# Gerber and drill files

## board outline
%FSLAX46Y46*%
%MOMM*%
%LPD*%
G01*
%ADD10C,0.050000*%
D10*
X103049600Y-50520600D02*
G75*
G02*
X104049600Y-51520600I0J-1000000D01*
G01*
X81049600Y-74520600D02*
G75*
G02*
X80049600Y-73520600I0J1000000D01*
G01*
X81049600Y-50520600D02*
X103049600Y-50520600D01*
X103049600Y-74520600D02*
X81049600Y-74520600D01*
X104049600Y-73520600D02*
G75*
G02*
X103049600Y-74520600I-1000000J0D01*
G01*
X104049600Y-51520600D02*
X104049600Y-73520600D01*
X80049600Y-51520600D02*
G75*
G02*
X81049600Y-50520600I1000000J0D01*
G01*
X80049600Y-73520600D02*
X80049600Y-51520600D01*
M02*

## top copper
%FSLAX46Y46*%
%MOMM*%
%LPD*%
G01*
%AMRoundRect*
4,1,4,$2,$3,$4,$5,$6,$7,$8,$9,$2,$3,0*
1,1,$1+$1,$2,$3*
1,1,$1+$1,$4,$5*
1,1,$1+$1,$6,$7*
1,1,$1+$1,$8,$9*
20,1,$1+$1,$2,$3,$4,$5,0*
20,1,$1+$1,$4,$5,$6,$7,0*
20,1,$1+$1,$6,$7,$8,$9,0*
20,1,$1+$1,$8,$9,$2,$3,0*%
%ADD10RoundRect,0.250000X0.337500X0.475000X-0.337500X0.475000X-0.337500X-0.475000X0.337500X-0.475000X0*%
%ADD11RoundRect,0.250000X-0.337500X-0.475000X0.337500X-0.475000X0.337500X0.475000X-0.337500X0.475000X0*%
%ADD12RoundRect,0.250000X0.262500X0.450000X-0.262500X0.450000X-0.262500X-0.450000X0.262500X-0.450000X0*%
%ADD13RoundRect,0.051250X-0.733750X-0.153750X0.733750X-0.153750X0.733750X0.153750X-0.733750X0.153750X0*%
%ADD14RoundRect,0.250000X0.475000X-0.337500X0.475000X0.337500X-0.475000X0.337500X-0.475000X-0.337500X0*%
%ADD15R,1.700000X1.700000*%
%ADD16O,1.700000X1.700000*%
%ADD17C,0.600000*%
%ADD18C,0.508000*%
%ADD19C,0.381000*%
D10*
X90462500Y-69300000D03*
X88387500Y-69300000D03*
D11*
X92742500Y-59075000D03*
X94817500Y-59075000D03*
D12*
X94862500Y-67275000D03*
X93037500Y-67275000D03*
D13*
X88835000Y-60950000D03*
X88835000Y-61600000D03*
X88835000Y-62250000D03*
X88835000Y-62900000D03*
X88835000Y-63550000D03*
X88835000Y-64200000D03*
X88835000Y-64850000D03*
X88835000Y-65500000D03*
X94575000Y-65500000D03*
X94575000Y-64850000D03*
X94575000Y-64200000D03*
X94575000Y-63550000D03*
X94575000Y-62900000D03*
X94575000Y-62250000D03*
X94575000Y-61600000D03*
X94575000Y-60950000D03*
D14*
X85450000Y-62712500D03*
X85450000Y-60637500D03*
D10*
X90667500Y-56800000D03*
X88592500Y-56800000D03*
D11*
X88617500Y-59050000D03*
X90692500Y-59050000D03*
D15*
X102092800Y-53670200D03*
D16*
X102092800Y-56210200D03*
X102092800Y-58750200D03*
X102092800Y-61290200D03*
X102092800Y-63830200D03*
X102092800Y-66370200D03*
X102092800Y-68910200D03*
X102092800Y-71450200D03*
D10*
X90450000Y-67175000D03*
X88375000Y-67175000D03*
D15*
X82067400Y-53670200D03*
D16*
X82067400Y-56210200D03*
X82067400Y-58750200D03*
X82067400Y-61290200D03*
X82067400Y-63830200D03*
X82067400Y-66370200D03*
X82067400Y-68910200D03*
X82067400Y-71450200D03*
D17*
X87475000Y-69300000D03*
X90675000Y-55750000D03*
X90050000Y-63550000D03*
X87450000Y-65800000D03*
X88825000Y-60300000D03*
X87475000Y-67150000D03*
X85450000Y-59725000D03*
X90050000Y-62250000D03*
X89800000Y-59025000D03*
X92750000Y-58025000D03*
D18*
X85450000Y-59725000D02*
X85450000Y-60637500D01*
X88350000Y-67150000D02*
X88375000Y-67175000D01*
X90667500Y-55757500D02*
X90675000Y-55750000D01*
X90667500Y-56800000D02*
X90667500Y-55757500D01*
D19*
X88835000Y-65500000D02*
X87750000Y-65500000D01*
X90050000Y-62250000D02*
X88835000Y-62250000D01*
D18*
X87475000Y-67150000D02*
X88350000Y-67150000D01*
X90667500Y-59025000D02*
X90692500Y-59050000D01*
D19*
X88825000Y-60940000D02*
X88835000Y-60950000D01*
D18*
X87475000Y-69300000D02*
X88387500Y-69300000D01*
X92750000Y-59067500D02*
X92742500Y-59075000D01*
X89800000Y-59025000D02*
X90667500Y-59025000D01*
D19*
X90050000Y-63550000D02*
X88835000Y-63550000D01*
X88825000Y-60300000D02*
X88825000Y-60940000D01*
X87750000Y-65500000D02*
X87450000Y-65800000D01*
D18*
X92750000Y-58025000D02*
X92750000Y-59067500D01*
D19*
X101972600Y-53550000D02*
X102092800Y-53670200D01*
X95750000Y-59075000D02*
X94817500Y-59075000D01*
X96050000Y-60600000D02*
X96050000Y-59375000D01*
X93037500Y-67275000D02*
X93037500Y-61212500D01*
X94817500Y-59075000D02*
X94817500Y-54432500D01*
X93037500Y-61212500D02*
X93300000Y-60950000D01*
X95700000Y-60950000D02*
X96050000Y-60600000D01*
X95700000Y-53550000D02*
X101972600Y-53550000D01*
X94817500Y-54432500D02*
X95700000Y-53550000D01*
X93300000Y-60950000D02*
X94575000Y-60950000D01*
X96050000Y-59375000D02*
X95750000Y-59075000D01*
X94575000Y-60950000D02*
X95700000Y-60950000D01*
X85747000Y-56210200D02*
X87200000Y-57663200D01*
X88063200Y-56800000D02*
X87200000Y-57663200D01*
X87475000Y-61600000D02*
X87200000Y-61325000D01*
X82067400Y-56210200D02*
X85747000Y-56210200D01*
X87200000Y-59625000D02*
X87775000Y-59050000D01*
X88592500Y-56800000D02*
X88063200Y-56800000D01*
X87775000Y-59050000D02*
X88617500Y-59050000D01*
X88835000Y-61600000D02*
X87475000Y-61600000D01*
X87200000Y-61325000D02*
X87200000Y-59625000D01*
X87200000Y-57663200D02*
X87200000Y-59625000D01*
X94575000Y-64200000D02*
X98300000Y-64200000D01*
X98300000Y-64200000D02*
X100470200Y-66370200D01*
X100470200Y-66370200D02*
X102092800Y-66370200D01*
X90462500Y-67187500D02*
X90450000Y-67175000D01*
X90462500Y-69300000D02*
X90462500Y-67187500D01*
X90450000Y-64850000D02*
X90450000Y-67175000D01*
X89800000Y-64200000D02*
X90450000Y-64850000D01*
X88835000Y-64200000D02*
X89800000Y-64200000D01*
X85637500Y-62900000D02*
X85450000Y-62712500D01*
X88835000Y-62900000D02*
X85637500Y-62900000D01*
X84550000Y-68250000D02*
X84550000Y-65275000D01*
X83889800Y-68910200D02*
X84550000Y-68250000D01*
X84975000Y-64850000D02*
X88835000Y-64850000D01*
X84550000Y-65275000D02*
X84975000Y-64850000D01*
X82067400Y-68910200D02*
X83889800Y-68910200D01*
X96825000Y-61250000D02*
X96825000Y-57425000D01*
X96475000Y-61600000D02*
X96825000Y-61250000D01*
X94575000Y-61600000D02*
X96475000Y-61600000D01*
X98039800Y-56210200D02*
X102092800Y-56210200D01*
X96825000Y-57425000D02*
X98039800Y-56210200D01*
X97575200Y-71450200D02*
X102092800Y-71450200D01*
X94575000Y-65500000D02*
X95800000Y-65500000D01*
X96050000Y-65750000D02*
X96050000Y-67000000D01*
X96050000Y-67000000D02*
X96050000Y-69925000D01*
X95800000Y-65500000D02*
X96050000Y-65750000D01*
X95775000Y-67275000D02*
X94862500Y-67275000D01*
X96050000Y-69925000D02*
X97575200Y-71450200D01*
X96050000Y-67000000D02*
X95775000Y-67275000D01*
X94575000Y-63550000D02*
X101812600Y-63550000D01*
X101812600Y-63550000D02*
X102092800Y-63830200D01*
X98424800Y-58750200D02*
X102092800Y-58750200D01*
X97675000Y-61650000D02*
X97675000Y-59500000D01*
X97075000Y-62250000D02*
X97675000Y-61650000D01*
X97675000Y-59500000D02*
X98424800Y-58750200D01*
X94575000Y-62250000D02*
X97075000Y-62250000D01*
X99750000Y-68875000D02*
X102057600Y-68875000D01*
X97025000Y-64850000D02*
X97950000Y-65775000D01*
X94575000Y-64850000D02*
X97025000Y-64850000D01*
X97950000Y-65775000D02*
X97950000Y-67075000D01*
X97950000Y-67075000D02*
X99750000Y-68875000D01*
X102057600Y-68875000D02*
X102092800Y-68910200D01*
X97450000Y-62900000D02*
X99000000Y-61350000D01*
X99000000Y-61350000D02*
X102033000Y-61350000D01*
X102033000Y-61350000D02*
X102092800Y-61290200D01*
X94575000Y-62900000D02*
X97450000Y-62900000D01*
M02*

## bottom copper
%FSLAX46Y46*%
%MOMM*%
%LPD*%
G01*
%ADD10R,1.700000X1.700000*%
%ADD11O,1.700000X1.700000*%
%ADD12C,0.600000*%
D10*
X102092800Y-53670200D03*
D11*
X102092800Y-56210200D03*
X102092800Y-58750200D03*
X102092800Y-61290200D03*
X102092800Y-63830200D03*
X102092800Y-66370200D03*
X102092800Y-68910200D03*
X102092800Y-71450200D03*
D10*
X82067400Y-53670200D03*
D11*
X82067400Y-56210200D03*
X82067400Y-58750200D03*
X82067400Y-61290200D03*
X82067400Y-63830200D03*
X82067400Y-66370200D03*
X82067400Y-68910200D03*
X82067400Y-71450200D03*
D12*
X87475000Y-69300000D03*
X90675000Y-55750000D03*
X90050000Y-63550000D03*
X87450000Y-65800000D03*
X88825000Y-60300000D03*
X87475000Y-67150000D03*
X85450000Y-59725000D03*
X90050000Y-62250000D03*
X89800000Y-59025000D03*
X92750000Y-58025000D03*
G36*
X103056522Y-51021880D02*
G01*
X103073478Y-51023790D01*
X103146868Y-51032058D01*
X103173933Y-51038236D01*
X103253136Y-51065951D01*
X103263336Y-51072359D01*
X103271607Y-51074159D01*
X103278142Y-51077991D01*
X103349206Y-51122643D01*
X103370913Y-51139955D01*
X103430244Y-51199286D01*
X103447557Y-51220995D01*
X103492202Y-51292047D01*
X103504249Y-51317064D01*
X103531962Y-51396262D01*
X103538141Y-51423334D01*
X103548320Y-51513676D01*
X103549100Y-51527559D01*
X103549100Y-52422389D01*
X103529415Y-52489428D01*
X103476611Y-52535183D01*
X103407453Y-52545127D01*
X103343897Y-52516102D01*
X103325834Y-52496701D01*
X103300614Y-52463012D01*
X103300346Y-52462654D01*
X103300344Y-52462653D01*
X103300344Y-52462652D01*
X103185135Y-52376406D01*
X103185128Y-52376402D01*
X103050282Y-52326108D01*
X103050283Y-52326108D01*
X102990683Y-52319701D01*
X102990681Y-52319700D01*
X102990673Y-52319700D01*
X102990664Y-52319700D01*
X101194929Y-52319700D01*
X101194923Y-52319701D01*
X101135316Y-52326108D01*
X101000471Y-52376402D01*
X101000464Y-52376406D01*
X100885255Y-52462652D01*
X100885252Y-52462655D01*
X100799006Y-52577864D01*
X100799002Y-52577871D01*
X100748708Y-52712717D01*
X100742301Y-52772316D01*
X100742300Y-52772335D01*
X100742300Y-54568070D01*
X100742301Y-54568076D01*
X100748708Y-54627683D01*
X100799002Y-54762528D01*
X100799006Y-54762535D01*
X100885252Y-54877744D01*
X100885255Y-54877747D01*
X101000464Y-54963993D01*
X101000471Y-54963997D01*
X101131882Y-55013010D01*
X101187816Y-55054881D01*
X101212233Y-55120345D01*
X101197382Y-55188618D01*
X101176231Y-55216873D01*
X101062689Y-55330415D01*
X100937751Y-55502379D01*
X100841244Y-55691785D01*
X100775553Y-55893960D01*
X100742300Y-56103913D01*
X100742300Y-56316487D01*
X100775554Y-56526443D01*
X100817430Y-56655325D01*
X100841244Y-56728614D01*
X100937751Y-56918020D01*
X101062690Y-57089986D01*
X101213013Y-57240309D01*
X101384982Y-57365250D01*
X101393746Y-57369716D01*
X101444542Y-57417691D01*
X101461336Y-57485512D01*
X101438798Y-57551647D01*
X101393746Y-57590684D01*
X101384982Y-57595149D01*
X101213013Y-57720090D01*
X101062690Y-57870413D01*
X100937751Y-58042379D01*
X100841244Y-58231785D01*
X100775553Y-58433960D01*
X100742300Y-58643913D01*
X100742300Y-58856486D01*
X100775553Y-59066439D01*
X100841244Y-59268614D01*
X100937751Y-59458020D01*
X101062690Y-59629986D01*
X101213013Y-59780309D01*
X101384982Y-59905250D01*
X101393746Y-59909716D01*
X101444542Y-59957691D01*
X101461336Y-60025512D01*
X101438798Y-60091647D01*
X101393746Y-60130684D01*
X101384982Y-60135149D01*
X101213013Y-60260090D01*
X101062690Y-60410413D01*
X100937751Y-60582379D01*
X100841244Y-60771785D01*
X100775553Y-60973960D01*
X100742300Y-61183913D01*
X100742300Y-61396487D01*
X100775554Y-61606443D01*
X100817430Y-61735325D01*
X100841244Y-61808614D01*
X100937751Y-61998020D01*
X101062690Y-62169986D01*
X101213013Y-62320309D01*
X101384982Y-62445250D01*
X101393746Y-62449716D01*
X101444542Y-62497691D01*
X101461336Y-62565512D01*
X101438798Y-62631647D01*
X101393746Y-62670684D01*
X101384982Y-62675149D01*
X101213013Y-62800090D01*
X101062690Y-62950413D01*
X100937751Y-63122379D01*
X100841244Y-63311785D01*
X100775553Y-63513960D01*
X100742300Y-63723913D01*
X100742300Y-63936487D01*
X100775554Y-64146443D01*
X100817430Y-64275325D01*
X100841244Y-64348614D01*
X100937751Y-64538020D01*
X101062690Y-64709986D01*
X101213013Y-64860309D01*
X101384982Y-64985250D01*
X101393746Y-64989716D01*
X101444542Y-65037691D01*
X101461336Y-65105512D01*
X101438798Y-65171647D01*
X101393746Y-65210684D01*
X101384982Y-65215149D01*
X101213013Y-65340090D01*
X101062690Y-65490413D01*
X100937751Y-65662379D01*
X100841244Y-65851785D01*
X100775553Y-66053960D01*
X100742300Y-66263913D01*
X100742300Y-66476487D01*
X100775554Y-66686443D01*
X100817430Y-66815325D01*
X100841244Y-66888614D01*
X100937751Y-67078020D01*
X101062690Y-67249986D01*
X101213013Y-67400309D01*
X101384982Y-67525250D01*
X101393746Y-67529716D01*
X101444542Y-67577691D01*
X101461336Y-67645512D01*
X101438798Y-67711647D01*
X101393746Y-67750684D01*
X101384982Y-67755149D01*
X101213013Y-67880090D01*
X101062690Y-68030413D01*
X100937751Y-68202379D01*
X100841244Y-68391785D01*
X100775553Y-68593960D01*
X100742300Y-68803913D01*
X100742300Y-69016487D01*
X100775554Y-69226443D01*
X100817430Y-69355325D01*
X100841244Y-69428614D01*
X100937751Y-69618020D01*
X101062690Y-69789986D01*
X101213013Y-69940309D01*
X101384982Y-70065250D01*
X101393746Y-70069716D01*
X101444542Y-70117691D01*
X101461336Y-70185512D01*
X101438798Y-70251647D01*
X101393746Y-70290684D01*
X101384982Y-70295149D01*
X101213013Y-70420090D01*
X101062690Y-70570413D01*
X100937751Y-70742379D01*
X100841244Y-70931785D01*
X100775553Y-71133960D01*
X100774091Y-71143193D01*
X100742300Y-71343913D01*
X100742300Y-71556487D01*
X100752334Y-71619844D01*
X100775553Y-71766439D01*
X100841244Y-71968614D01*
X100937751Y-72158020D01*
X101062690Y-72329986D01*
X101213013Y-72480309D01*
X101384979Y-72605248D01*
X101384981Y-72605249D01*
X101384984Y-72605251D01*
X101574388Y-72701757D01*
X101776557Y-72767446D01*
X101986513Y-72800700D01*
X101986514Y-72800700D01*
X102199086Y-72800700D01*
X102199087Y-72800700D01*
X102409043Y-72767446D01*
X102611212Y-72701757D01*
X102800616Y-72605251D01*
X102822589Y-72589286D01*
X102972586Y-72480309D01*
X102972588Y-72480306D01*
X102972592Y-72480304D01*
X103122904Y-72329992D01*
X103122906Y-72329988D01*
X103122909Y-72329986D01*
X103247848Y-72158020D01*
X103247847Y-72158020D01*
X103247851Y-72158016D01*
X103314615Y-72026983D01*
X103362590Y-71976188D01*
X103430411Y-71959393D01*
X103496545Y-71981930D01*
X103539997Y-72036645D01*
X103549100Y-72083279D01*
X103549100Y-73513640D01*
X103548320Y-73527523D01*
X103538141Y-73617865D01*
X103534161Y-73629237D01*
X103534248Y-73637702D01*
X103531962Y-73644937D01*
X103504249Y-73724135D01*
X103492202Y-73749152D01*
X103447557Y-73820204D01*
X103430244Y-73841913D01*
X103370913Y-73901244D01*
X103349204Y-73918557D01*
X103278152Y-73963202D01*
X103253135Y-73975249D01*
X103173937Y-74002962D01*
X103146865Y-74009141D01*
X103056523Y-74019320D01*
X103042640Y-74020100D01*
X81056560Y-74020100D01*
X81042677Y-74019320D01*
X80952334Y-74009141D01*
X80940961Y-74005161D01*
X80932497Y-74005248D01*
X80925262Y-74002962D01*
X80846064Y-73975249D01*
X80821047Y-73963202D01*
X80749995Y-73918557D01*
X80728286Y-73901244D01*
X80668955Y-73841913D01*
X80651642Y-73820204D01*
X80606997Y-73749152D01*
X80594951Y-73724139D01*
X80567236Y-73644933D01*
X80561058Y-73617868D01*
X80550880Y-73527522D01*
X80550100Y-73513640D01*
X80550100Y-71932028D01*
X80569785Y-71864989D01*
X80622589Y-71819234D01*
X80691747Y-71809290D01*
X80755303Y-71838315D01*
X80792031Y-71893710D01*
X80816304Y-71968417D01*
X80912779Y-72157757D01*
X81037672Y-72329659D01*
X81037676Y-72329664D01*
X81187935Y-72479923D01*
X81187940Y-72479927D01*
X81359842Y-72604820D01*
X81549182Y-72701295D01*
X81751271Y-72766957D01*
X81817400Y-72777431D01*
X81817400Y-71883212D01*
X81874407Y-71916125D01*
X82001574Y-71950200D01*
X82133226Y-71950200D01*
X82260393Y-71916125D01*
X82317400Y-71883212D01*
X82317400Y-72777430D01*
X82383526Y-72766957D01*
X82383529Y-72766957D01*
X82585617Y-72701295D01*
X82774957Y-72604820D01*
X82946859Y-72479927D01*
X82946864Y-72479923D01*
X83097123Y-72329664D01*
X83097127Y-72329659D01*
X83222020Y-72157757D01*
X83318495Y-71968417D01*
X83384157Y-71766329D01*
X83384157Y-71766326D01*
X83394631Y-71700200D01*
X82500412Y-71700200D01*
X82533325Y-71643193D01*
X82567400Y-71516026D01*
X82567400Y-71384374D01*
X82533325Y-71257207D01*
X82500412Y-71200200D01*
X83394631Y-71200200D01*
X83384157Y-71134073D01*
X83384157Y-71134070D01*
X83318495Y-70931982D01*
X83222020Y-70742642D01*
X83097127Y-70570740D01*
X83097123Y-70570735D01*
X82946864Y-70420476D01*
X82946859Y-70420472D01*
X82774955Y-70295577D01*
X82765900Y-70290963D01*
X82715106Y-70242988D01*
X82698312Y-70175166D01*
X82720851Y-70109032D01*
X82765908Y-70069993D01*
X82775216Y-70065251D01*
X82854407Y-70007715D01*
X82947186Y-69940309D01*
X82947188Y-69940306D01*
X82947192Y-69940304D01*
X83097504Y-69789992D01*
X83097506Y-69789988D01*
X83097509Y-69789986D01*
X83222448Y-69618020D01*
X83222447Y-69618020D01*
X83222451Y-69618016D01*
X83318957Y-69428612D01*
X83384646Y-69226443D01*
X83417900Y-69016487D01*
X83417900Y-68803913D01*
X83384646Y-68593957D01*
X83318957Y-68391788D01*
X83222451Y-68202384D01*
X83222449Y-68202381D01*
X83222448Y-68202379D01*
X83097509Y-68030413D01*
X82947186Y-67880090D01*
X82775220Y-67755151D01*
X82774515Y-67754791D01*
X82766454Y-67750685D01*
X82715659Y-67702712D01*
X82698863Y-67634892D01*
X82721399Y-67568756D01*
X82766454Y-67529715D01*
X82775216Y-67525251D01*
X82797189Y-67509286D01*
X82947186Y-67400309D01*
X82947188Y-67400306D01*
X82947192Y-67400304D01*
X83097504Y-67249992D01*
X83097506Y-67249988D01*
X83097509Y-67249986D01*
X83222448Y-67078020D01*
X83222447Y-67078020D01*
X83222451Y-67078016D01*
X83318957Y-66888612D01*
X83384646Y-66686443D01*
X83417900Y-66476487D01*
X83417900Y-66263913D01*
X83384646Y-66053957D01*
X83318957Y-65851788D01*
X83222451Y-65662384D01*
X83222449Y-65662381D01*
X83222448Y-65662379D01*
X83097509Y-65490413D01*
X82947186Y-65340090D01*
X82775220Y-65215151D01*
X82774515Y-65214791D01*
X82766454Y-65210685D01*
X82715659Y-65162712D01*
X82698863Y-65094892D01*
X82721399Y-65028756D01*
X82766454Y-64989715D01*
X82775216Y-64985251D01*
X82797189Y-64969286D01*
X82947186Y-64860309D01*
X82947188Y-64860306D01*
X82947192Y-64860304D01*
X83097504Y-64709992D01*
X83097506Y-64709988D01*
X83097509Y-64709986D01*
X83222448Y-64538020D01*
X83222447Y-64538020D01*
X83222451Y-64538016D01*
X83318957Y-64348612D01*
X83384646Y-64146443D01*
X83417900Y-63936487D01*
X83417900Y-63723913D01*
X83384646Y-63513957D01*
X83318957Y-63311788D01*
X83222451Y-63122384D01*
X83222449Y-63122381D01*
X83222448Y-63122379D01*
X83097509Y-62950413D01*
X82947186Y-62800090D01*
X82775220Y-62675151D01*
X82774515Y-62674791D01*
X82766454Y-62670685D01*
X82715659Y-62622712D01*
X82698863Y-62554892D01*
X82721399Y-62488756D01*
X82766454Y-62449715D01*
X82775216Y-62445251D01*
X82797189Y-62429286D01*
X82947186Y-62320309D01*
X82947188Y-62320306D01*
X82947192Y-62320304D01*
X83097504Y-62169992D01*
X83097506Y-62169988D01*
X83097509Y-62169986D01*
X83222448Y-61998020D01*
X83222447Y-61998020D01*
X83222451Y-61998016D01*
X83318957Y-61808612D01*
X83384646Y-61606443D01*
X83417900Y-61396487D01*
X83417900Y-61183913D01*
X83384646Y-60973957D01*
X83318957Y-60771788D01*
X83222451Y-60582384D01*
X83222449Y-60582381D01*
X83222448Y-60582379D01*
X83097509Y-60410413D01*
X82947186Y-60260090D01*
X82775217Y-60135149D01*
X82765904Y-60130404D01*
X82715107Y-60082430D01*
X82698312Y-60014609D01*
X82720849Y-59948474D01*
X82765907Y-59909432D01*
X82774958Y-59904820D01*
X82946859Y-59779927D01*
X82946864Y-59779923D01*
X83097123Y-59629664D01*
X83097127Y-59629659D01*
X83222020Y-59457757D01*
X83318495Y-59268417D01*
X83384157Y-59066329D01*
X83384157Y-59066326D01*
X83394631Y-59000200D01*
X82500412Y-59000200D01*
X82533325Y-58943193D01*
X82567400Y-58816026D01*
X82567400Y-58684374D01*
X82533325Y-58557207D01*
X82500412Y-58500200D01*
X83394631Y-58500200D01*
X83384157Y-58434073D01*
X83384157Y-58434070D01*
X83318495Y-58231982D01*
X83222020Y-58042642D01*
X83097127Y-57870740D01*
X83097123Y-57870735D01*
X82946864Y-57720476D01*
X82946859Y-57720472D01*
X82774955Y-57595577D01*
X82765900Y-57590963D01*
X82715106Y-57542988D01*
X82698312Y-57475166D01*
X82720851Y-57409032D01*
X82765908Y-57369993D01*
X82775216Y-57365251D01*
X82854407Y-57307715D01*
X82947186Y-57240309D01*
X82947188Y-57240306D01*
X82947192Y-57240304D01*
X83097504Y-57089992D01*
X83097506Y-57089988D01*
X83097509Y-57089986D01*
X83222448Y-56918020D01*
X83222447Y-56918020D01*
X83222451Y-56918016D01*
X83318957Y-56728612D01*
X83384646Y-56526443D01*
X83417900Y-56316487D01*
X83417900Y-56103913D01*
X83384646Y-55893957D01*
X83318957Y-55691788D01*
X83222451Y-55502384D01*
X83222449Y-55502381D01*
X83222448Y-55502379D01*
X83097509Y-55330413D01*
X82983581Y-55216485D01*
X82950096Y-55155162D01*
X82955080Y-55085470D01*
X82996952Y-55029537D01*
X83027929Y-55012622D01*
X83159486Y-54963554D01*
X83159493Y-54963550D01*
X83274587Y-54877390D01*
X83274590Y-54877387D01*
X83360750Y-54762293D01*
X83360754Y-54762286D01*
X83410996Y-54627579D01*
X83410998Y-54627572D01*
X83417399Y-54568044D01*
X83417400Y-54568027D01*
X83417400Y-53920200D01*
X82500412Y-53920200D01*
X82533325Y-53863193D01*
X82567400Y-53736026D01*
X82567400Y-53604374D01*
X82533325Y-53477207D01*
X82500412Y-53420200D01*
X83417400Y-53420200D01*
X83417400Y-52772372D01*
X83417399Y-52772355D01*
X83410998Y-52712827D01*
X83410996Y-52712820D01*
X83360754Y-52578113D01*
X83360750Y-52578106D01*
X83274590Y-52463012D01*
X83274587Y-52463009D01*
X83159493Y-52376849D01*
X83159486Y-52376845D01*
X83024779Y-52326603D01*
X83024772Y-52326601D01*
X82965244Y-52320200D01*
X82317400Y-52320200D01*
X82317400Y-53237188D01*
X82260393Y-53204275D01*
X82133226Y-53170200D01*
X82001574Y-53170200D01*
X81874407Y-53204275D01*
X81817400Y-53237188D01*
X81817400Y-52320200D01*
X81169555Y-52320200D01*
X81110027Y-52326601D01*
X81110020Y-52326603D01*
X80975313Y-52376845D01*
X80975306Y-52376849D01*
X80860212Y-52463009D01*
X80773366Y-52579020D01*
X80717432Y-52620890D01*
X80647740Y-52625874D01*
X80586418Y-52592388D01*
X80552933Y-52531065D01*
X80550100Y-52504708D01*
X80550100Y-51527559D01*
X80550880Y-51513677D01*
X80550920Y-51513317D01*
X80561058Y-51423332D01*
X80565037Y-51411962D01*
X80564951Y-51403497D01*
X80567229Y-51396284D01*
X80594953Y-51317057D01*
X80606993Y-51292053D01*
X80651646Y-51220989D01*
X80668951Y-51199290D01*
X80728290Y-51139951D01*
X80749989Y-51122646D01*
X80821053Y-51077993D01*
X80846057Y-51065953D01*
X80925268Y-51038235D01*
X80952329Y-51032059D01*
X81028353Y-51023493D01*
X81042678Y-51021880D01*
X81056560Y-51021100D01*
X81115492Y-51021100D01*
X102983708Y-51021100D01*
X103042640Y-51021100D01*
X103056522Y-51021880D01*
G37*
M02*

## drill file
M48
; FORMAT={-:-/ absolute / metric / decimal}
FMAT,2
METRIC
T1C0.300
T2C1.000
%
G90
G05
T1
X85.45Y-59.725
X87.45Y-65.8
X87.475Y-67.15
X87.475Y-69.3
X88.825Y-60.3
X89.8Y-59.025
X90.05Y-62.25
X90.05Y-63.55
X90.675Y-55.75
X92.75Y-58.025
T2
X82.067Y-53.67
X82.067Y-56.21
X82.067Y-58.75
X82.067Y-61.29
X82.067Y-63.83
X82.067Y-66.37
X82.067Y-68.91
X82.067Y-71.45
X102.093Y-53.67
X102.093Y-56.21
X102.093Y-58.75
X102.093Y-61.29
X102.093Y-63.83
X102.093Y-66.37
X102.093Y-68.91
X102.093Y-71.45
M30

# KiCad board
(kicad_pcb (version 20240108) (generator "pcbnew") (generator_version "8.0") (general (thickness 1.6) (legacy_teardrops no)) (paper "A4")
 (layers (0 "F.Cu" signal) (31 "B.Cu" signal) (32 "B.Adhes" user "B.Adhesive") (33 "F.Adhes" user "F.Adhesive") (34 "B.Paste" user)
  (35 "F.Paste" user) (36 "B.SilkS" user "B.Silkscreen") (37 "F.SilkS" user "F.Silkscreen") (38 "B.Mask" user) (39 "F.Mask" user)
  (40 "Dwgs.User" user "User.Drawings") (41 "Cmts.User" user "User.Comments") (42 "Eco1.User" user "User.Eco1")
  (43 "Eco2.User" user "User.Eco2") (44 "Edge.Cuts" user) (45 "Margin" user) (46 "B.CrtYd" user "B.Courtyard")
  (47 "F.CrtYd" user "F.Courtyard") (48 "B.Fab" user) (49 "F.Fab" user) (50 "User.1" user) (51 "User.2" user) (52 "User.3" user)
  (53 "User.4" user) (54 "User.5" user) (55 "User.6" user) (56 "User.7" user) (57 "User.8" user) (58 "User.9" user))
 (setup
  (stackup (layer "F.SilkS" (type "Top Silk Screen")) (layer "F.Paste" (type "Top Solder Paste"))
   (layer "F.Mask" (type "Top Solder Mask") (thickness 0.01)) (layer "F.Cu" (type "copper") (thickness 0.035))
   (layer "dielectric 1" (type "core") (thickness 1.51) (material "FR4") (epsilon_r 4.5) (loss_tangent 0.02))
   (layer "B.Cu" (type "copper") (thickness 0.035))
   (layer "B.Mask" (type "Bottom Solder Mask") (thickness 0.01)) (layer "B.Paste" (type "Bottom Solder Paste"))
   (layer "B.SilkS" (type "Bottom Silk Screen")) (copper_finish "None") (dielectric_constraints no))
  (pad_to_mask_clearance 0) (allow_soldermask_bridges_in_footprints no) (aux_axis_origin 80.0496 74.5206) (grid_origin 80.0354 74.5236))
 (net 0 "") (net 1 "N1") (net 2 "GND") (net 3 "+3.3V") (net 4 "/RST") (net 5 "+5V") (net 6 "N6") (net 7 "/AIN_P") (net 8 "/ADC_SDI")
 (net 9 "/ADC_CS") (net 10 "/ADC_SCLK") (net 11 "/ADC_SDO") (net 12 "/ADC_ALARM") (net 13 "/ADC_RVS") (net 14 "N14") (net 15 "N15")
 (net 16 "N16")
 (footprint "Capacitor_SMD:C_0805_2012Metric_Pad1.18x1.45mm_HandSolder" (layer "F.Cu") (at 89.425 69.3 180)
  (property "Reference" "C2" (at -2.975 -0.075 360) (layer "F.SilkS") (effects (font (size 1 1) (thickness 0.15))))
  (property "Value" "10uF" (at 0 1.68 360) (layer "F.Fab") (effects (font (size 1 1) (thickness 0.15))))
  (pad "1" smd roundrect (at -1.0375 0 180) (size 1.175 1.45) (layers "F.Cu" "F.Paste" "F.Mask") (roundrect_rratio 0.212766) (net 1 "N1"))
  (pad "2" smd roundrect (at 1.0375 0 180) (size 1.175 1.45) (layers "F.Cu" "F.Paste" "F.Mask") (roundrect_rratio 0.212766) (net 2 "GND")))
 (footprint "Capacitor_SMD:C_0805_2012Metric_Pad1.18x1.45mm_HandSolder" (layer "F.Cu") (at 93.78 59.075)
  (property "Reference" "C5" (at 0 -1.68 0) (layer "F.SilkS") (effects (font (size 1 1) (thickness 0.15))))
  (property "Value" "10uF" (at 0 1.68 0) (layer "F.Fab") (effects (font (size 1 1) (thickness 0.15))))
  (pad "1" smd roundrect (at -1.0375 0) (size 1.175 1.45) (layers "F.Cu" "F.Paste" "F.Mask") (roundrect_rratio 0.212766) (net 2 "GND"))
  (pad "2" smd roundrect (at 1.0375 0) (size 1.175 1.45) (layers "F.Cu" "F.Paste" "F.Mask") (roundrect_rratio 0.212766) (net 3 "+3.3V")))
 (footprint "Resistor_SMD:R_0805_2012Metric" (layer "F.Cu") (at 93.95 67.275 180)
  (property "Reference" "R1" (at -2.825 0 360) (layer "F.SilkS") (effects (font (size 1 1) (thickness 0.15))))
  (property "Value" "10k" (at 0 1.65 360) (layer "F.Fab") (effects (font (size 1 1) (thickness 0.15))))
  (pad "1" smd roundrect (at -0.9125 0 180) (size 1.025 1.4) (layers "F.Cu" "F.Paste" "F.Mask") (roundrect_rratio 0.243902) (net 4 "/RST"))
  (pad "2" smd roundrect (at 0.9125 0 180) (size 1.025 1.4) (layers "F.Cu" "F.Paste" "F.Mask") (roundrect_rratio 0.243902) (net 3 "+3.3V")))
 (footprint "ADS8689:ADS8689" (layer "F.Cu") (at 91.705 63.225)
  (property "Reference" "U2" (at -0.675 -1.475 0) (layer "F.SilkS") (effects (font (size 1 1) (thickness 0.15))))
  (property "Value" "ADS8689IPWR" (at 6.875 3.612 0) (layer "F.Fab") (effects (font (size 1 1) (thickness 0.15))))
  (pad "1" smd roundrect (at -2.87 -2.275) (size 1.57 0.41) (layers "F.Cu" "F.Paste" "F.Mask") (roundrect_rratio 0.125) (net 2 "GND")
   (solder_mask_margin 0.102))
  (pad "2" smd roundrect (at -2.87 -1.625) (size 1.57 0.41) (layers "F.Cu" "F.Paste" "F.Mask") (roundrect_rratio 0.125) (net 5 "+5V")
   (solder_mask_margin 0.102))
  (pad "3" smd roundrect (at -2.87 -0.975) (size 1.57 0.41) (layers "F.Cu" "F.Paste" "F.Mask") (roundrect_rratio 0.125) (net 2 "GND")
   (solder_mask_margin 0.102))
  (pad "4" smd roundrect (at -2.87 -0.325) (size 1.57 0.41) (layers "F.Cu" "F.Paste" "F.Mask") (roundrect_rratio 0.125) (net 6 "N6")
   (solder_mask_margin 0.102))
  (pad "5" smd roundrect (at -2.87 0.325) (size 1.57 0.41) (layers "F.Cu" "F.Paste" "F.Mask") (roundrect_rratio 0.125) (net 2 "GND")
   (solder_mask_margin 0.102))
  (pad "6" smd roundrect (at -2.87 0.975) (size 1.57 0.41) (layers "F.Cu" "F.Paste" "F.Mask") (roundrect_rratio 0.125) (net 1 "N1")
   (solder_mask_margin 0.102))
  (pad "7" smd roundrect (at -2.87 1.625) (size 1.57 0.41) (layers "F.Cu" "F.Paste" "F.Mask") (roundrect_rratio 0.125) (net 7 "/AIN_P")
   (solder_mask_margin 0.102))
  (pad "8" smd roundrect (at -2.87 2.275) (size 1.57 0.41) (layers "F.Cu" "F.Paste" "F.Mask") (roundrect_rratio 0.125) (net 2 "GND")
   (solder_mask_margin 0.102))
  (pad "9" smd roundrect (at 2.87 2.275) (size 1.57 0.41) (layers "F.Cu" "F.Paste" "F.Mask") (roundrect_rratio 0.125) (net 4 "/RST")
   (solder_mask_margin 0.102))
  (pad "10" smd roundrect (at 2.87 1.625) (size 1.57 0.41) (layers "F.Cu" "F.Paste" "F.Mask") (roundrect_rratio 0.125) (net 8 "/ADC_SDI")
   (solder_mask_margin 0.102))
  (pad "11" smd roundrect (at 2.87 0.975) (size 1.57 0.41) (layers "F.Cu" "F.Paste" "F.Mask") (roundrect_rratio 0.125) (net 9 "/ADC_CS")
   (solder_mask_margin 0.102))
  (pad "12" smd roundrect (at 2.87 0.325) (size 1.57 0.41) (layers "F.Cu" "F.Paste" "F.Mask") (roundrect_rratio 0.125) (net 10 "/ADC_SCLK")
   (solder_mask_margin 0.102))
  (pad "13" smd roundrect (at 2.87 -0.325) (size 1.57 0.41) (layers "F.Cu" "F.Paste" "F.Mask") (roundrect_rratio 0.125) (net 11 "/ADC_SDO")
   (solder_mask_margin 0.102))
  (pad "14" smd roundrect (at 2.87 -0.975) (size 1.57 0.41) (layers "F.Cu" "F.Paste" "F.Mask") (roundrect_rratio 0.125)
   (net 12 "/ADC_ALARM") (solder_mask_margin 0.102))
  (pad "15" smd roundrect (at 2.87 -1.625) (size 1.57 0.41) (layers "F.Cu" "F.Paste" "F.Mask") (roundrect_rratio 0.125) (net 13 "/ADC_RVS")
   (solder_mask_margin 0.102))
  (pad "16" smd roundrect (at 2.87 -2.275) (size 1.57 0.41) (layers "F.Cu" "F.Paste" "F.Mask") (roundrect_rratio 0.125) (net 3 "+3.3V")
   (solder_mask_margin 0.102)))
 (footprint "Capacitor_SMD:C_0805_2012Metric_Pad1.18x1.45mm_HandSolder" (layer "F.Cu") (at 85.45 61.675 90)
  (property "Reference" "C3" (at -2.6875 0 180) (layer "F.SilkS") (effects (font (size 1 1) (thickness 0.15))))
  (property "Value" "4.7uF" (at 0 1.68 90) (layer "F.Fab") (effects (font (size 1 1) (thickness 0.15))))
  (pad "1" smd roundrect (at -1.0375 0 90) (size 1.175 1.45) (layers "F.Cu" "F.Paste" "F.Mask") (roundrect_rratio 0.212766) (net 6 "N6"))
  (pad "2" smd roundrect (at 1.0375 0 90) (size 1.175 1.45) (layers "F.Cu" "F.Paste" "F.Mask") (roundrect_rratio 0.212766) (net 2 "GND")))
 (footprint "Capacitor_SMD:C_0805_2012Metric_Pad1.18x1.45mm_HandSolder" (layer "F.Cu") (at 89.63 56.8 180)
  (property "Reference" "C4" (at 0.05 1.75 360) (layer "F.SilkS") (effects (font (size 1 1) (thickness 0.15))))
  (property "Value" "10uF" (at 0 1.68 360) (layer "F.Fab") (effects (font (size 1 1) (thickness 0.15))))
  (pad "1" smd roundrect (at -1.0375 0 180) (size 1.175 1.45) (layers "F.Cu" "F.Paste" "F.Mask") (roundrect_rratio 0.212766) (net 2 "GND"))
  (pad "2" smd roundrect (at 1.0375 0 180) (size 1.175 1.45) (layers "F.Cu" "F.Paste" "F.Mask") (roundrect_rratio 0.212766) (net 5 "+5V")))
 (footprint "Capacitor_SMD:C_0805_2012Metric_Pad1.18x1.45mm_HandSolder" (layer "F.Cu") (at 89.655 59.05)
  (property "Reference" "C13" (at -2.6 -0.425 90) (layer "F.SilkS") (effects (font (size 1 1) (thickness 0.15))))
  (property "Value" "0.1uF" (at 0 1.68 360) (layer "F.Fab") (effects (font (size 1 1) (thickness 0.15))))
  (pad "1" smd roundrect (at -1.0375 0) (size 1.175 1.45) (layers "F.Cu" "F.Paste" "F.Mask") (roundrect_rratio 0.212766) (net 5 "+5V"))
  (pad "2" smd roundrect (at 1.0375 0) (size 1.175 1.45) (layers "F.Cu" "F.Paste" "F.Mask") (roundrect_rratio 0.212766) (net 2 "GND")))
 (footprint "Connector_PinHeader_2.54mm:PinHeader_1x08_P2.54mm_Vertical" (layer "F.Cu") (at 102.0928 53.6702)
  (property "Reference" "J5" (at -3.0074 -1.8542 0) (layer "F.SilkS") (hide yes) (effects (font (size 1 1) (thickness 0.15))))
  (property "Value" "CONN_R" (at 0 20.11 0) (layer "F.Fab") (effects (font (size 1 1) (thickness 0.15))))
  (pad "1" thru_hole rect (at 0 0) (size 1.7 1.7) (drill 1) (layers "*.Cu" "*.Mask") (remove_unused_layers no) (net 3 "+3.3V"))
  (pad "2" thru_hole oval (at 0 2.54) (size 1.7 1.7) (drill 1) (layers "*.Cu" "*.Mask") (remove_unused_layers no) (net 13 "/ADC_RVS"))
  (pad "3" thru_hole oval (at 0 5.08) (size 1.7 1.7) (drill 1) (layers "*.Cu" "*.Mask") (remove_unused_layers no) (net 12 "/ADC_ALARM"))
  (pad "4" thru_hole oval (at 0 7.62) (size 1.7 1.7) (drill 1) (layers "*.Cu" "*.Mask") (remove_unused_layers no) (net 11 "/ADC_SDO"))
  (pad "5" thru_hole oval (at 0 10.16) (size 1.7 1.7) (drill 1) (layers "*.Cu" "*.Mask") (remove_unused_layers no) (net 10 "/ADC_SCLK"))
  (pad "6" thru_hole oval (at 0 12.7) (size 1.7 1.7) (drill 1) (layers "*.Cu" "*.Mask") (remove_unused_layers no) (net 9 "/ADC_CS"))
  (pad "7" thru_hole oval (at 0 15.24) (size 1.7 1.7) (drill 1) (layers "*.Cu" "*.Mask") (remove_unused_layers no) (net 8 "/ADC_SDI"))
  (pad "8" thru_hole oval (at 0 17.78) (size 1.7 1.7) (drill 1) (layers "*.Cu" "*.Mask") (remove_unused_layers no) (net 4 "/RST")))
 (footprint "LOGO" (layer "F.Cu") (at 96.125 54.1)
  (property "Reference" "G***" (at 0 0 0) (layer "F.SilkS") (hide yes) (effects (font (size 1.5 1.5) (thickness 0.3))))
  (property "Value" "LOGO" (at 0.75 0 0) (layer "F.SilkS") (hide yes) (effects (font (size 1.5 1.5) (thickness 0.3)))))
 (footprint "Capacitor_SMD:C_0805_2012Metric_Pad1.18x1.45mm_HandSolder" (layer "F.Cu") (at 89.4125 67.175 180)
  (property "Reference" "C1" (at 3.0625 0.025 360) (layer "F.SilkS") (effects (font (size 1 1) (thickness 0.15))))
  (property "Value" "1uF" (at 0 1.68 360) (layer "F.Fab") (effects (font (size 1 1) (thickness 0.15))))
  (pad "1" smd roundrect (at -1.0375 0 180) (size 1.175 1.45) (layers "F.Cu" "F.Paste" "F.Mask") (roundrect_rratio 0.212766) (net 1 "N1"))
  (pad "2" smd roundrect (at 1.0375 0 180) (size 1.175 1.45) (layers "F.Cu" "F.Paste" "F.Mask") (roundrect_rratio 0.212766) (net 2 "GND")))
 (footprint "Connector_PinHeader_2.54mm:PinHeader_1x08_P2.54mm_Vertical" (layer "F.Cu") (at 82.0674 53.6702)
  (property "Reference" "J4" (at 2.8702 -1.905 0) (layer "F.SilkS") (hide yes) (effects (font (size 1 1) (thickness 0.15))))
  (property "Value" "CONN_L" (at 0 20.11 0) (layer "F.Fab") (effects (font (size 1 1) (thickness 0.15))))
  (pad "1" thru_hole rect (at 0 0) (size 1.7 1.7) (drill 1) (layers "*.Cu" "*.Mask") (remove_unused_layers no) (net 2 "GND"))
  (pad "2" thru_hole oval (at 0 2.54) (size 1.7 1.7) (drill 1) (layers "*.Cu" "*.Mask") (remove_unused_layers no) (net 5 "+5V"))
  (pad "3" thru_hole oval (at 0 5.08) (size 1.7 1.7) (drill 1) (layers "*.Cu" "*.Mask") (remove_unused_layers no) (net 2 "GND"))
  (pad "4" thru_hole oval (at 0 7.62) (size 1.7 1.7) (drill 1) (layers "*.Cu" "*.Mask") (remove_unused_layers no) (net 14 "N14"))
  (pad "5" thru_hole oval (at 0 10.16) (size 1.7 1.7) (drill 1) (layers "*.Cu" "*.Mask") (remove_unused_layers no) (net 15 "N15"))
  (pad "6" thru_hole oval (at 0 12.7) (size 1.7 1.7) (drill 1) (layers "*.Cu" "*.Mask") (remove_unused_layers no) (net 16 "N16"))
  (pad "7" thru_hole oval (at 0 15.24) (size 1.7 1.7) (drill 1) (layers "*.Cu" "*.Mask") (remove_unused_layers no) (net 7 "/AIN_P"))
  (pad "8" thru_hole oval (at 0 17.78) (size 1.7 1.7) (drill 1) (layers "*.Cu" "*.Mask") (remove_unused_layers no) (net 2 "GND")))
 (gr_arc (start 103.0496 50.5206) (mid 103.756707 50.813493) (end 104.0496 51.5206) (stroke (width 0.05) (type default)) (layer "Edge.Cuts"))
 (gr_arc (start 81.0496 74.5206) (mid 80.342493 74.227707) (end 80.0496 73.5206) (stroke (width 0.05) (type default)) (layer "Edge.Cuts"))
 (gr_line (start 81.0496 50.5206) (end 103.0496 50.5206) (stroke (width 0.05) (type default)) (layer "Edge.Cuts"))
 (gr_line (start 103.0496 74.5206) (end 81.0496 74.5206) (stroke (width 0.05) (type default)) (layer "Edge.Cuts"))
 (gr_arc (start 104.0496 73.5206) (mid 103.756707 74.227707) (end 103.0496 74.5206) (stroke (width 0.05) (type default)) (layer "Edge.Cuts"))
 (gr_line (start 104.0496 51.5206) (end 104.0496 73.5206) (stroke (width 0.05) (type default)) (layer "Edge.Cuts"))
 (gr_arc (start 80.0496 51.5206) (mid 80.342493 50.813493) (end 81.0496 50.5206) (stroke (width 0.05) (type default)) (layer "Edge.Cuts"))
 (gr_line (start 80.0496 73.5206) (end 80.0496 51.5206) (stroke (width 0.05) (type default)) (layer "Edge.Cuts"))
 (segment (start 85.45 59.725) (end 85.45 60.6375) (width 0.508) (layer "F.Cu") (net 2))
 (segment (start 88.35 67.15) (end 88.375 67.175) (width 0.508) (layer "F.Cu") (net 2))
 (segment (start 90.6675 55.7575) (end 90.675 55.75) (width 0.508) (layer "F.Cu") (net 2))
 (segment (start 90.6675 56.8) (end 90.6675 55.7575) (width 0.508) (layer "F.Cu") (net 2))
 (segment (start 88.835 65.5) (end 87.75 65.5) (width 0.381) (layer "F.Cu") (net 2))
 (segment (start 90.05 62.25) (end 88.835 62.25) (width 0.381) (layer "F.Cu") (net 2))
 (segment (start 87.475 67.15) (end 88.35 67.15) (width 0.508) (layer "F.Cu") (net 2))
 (segment (start 90.6675 59.025) (end 90.6925 59.05) (width 0.508) (layer "F.Cu") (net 2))
 (segment (start 88.825 60.94) (end 88.835 60.95) (width 0.381) (layer "F.Cu") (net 2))
 (segment (start 87.475 69.3) (end 88.3875 69.3) (width 0.508) (layer "F.Cu") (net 2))
 (segment (start 92.75 59.0675) (end 92.7425 59.075) (width 0.508) (layer "F.Cu") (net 2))
 (segment (start 89.8 59.025) (end 90.6675 59.025) (width 0.508) (layer "F.Cu") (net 2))
 (segment (start 90.05 63.55) (end 88.835 63.55) (width 0.381) (layer "F.Cu") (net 2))
 (segment (start 88.825 60.3) (end 88.825 60.94) (width 0.381) (layer "F.Cu") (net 2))
 (segment (start 87.75 65.5) (end 87.45 65.8) (width 0.381) (layer "F.Cu") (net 2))
 (segment (start 92.75 58.025) (end 92.75 59.0675) (width 0.508) (layer "F.Cu") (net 2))
 (via (at 87.475 69.3) (size 0.6) (drill 0.3) (layers "F.Cu" "B.Cu") (free yes) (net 2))
 (via (at 90.675 55.75) (size 0.6) (drill 0.3) (layers "F.Cu" "B.Cu") (free yes) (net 2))
 (via (at 90.05 63.55) (size 0.6) (drill 0.3) (layers "F.Cu" "B.Cu") (free yes) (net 2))
 (via (at 87.45 65.8) (size 0.6) (drill 0.3) (layers "F.Cu" "B.Cu") (free yes) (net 2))
 (via (at 88.825 60.3) (size 0.6) (drill 0.3) (layers "F.Cu" "B.Cu") (free yes) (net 2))
 (via (at 87.475 67.15) (size 0.6) (drill 0.3) (layers "F.Cu" "B.Cu") (free yes) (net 2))
 (via (at 85.45 59.725) (size 0.6) (drill 0.3) (layers "F.Cu" "B.Cu") (free yes) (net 2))
 (via (at 90.05 62.25) (size 0.6) (drill 0.3) (layers "F.Cu" "B.Cu") (free yes) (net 2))
 (via (at 89.8 59.025) (size 0.6) (drill 0.3) (layers "F.Cu" "B.Cu") (free yes) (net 2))
 (via (at 92.75 58.025) (size 0.6) (drill 0.3) (layers "F.Cu" "B.Cu") (free yes) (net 2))
 (segment (start 101.9726 53.55) (end 102.0928 53.6702) (width 0.381) (layer "F.Cu") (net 3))
 (segment (start 95.75 59.075) (end 94.8175 59.075) (width 0.381) (layer "F.Cu") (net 3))
 (segment (start 96.05 60.6) (end 96.05 59.375) (width 0.381) (layer "F.Cu") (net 3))
 (segment (start 93.0375 67.275) (end 93.0375 61.2125) (width 0.381) (layer "F.Cu") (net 3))
 (segment (start 94.8175 59.075) (end 94.8175 54.4325) (width 0.381) (layer "F.Cu") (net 3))
 (segment (start 93.0375 61.2125) (end 93.3 60.95) (width 0.381) (layer "F.Cu") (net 3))
 (segment (start 95.7 60.95) (end 96.05 60.6) (width 0.381) (layer "F.Cu") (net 3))
 (segment (start 95.7 53.55) (end 101.9726 53.55) (width 0.381) (layer "F.Cu") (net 3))
 (segment (start 94.8175 54.4325) (end 95.7 53.55) (width 0.381) (layer "F.Cu") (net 3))
 (segment (start 93.3 60.95) (end 94.575 60.95) (width 0.381) (layer "F.Cu") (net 3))
 (segment (start 96.05 59.375) (end 95.75 59.075) (width 0.381) (layer "F.Cu") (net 3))
 (segment (start 94.575 60.95) (end 95.7 60.95) (width 0.381) (layer "F.Cu") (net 3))
 (segment (start 85.747 56.2102) (end 87.2 57.6632) (width 0.381) (layer "F.Cu") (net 5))
 (segment (start 88.0632 56.8) (end 87.2 57.6632) (width 0.381) (layer "F.Cu") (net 5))
 (segment (start 87.475 61.6) (end 87.2 61.325) (width 0.381) (layer "F.Cu") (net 5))
 (segment (start 82.0674 56.2102) (end 85.747 56.2102) (width 0.381) (layer "F.Cu") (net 5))
 (segment (start 87.2 59.625) (end 87.775 59.05) (width 0.381) (layer "F.Cu") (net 5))
 (segment (start 88.5925 56.8) (end 88.0632 56.8) (width 0.381) (layer "F.Cu") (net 5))
 (segment (start 87.775 59.05) (end 88.6175 59.05) (width 0.381) (layer "F.Cu") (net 5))
 (segment (start 88.835 61.6) (end 87.475 61.6) (width 0.381) (layer "F.Cu") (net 5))
 (segment (start 87.2 61.325) (end 87.2 59.625) (width 0.381) (layer "F.Cu") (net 5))
 (segment (start 87.2 57.6632) (end 87.2 59.625) (width 0.381) (layer "F.Cu") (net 5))
 (segment (start 94.575 64.2) (end 98.3 64.2) (width 0.381) (layer "F.Cu") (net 9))
 (segment (start 98.3 64.2) (end 100.4702 66.3702) (width 0.381) (layer "F.Cu") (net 9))
 (segment (start 100.4702 66.3702) (end 102.0928 66.3702) (width 0.381) (layer "F.Cu") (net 9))
 (segment (start 90.4625 67.1875) (end 90.45 67.175) (width 0.381) (layer "F.Cu") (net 1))
 (segment (start 90.4625 69.3) (end 90.4625 67.1875) (width 0.381) (layer "F.Cu") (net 1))
 (segment (start 90.45 64.85) (end 90.45 67.175) (width 0.381) (layer "F.Cu") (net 1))
 (segment (start 89.8 64.2) (end 90.45 64.85) (width 0.381) (layer "F.Cu") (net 1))
 (segment (start 88.835 64.2) (end 89.8 64.2) (width 0.381) (layer "F.Cu") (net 1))
 (segment (start 85.6375 62.9) (end 85.45 62.7125) (width 0.381) (layer "F.Cu") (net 6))
 (segment (start 88.835 62.9) (end 85.6375 62.9) (width 0.381) (layer "F.Cu") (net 6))
 (segment (start 84.55 68.25) (end 84.55 65.275) (width 0.381) (layer "F.Cu") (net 7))
 (segment (start 83.8898 68.9102) (end 84.55 68.25) (width 0.381) (layer "F.Cu") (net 7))
 (segment (start 84.975 64.85) (end 88.835 64.85) (width 0.381) (layer "F.Cu") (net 7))
 (segment (start 84.55 65.275) (end 84.975 64.85) (width 0.381) (layer "F.Cu") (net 7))
 (segment (start 82.0674 68.9102) (end 83.8898 68.9102) (width 0.381) (layer "F.Cu") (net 7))
 (segment (start 96.825 61.25) (end 96.825 57.425) (width 0.381) (layer "F.Cu") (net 13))
 (segment (start 96.475 61.6) (end 96.825 61.25) (width 0.381) (layer "F.Cu") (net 13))
 (segment (start 94.575 61.6) (end 96.475 61.6) (width 0.381) (layer "F.Cu") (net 13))
 (segment (start 98.0398 56.2102) (end 102.0928 56.2102) (width 0.381) (layer "F.Cu") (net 13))
 (segment (start 96.825 57.425) (end 98.0398 56.2102) (width 0.381) (layer "F.Cu") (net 13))
 (segment (start 97.5752 71.4502) (end 102.0928 71.4502) (width 0.381) (layer "F.Cu") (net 4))
 (segment (start 94.575 65.5) (end 95.8 65.5) (width 0.381) (layer "F.Cu") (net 4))
 (segment (start 96.05 65.75) (end 96.05 67) (width 0.381) (layer "F.Cu") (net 4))
 (segment (start 96.05 67) (end 96.05 69.925) (width 0.381) (layer "F.Cu") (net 4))
 (segment (start 95.8 65.5) (end 96.05 65.75) (width 0.381) (layer "F.Cu") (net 4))
 (segment (start 95.775 67.275) (end 94.8625 67.275) (width 0.381) (layer "F.Cu") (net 4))
 (segment (start 96.05 69.925) (end 97.5752 71.4502) (width 0.381) (layer "F.Cu") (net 4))
 (segment (start 96.05 67) (end 95.775 67.275) (width 0.381) (layer "F.Cu") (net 4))
 (segment (start 94.575 63.55) (end 101.8126 63.55) (width 0.381) (layer "F.Cu") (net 10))
 (segment (start 101.8126 63.55) (end 102.0928 63.8302) (width 0.381) (layer "F.Cu") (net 10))
 (segment (start 98.4248 58.7502) (end 102.0928 58.7502) (width 0.381) (layer "F.Cu") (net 12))
 (segment (start 97.675 61.65) (end 97.675 59.5) (width 0.381) (layer "F.Cu") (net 12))
 (segment (start 97.075 62.25) (end 97.675 61.65) (width 0.381) (layer "F.Cu") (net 12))
 (segment (start 97.675 59.5) (end 98.4248 58.7502) (width 0.381) (layer "F.Cu") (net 12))
 (segment (start 94.575 62.25) (end 97.075 62.25) (width 0.381) (layer "F.Cu") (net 12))
 (segment (start 99.75 68.875) (end 102.0576 68.875) (width 0.381) (layer "F.Cu") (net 8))
 (segment (start 97.025 64.85) (end 97.95 65.775) (width 0.381) (layer "F.Cu") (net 8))
 (segment (start 94.575 64.85) (end 97.025 64.85) (width 0.381) (layer "F.Cu") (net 8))
 (segment (start 97.95 65.775) (end 97.95 67.075) (width 0.381) (layer "F.Cu") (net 8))
 (segment (start 97.95 67.075) (end 99.75 68.875) (width 0.381) (layer "F.Cu") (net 8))
 (segment (start 102.0576 68.875) (end 102.0928 68.9102) (width 0.381) (layer "F.Cu") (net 8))
 (segment (start 97.45 62.9) (end 99 61.35) (width 0.381) (layer "F.Cu") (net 11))
 (segment (start 99 61.35) (end 102.033 61.35) (width 0.381) (layer "F.Cu") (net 11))
 (segment (start 102.033 61.35) (end 102.0928 61.2902) (width 0.381) (layer "F.Cu") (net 11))
 (segment (start 94.575 62.9) (end 97.45 62.9) (width 0.381) (layer "F.Cu") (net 11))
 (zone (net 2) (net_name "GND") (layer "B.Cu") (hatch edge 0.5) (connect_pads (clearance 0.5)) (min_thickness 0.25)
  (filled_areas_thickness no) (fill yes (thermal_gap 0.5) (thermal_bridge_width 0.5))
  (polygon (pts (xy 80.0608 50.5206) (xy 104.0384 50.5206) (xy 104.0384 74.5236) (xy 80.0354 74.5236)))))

